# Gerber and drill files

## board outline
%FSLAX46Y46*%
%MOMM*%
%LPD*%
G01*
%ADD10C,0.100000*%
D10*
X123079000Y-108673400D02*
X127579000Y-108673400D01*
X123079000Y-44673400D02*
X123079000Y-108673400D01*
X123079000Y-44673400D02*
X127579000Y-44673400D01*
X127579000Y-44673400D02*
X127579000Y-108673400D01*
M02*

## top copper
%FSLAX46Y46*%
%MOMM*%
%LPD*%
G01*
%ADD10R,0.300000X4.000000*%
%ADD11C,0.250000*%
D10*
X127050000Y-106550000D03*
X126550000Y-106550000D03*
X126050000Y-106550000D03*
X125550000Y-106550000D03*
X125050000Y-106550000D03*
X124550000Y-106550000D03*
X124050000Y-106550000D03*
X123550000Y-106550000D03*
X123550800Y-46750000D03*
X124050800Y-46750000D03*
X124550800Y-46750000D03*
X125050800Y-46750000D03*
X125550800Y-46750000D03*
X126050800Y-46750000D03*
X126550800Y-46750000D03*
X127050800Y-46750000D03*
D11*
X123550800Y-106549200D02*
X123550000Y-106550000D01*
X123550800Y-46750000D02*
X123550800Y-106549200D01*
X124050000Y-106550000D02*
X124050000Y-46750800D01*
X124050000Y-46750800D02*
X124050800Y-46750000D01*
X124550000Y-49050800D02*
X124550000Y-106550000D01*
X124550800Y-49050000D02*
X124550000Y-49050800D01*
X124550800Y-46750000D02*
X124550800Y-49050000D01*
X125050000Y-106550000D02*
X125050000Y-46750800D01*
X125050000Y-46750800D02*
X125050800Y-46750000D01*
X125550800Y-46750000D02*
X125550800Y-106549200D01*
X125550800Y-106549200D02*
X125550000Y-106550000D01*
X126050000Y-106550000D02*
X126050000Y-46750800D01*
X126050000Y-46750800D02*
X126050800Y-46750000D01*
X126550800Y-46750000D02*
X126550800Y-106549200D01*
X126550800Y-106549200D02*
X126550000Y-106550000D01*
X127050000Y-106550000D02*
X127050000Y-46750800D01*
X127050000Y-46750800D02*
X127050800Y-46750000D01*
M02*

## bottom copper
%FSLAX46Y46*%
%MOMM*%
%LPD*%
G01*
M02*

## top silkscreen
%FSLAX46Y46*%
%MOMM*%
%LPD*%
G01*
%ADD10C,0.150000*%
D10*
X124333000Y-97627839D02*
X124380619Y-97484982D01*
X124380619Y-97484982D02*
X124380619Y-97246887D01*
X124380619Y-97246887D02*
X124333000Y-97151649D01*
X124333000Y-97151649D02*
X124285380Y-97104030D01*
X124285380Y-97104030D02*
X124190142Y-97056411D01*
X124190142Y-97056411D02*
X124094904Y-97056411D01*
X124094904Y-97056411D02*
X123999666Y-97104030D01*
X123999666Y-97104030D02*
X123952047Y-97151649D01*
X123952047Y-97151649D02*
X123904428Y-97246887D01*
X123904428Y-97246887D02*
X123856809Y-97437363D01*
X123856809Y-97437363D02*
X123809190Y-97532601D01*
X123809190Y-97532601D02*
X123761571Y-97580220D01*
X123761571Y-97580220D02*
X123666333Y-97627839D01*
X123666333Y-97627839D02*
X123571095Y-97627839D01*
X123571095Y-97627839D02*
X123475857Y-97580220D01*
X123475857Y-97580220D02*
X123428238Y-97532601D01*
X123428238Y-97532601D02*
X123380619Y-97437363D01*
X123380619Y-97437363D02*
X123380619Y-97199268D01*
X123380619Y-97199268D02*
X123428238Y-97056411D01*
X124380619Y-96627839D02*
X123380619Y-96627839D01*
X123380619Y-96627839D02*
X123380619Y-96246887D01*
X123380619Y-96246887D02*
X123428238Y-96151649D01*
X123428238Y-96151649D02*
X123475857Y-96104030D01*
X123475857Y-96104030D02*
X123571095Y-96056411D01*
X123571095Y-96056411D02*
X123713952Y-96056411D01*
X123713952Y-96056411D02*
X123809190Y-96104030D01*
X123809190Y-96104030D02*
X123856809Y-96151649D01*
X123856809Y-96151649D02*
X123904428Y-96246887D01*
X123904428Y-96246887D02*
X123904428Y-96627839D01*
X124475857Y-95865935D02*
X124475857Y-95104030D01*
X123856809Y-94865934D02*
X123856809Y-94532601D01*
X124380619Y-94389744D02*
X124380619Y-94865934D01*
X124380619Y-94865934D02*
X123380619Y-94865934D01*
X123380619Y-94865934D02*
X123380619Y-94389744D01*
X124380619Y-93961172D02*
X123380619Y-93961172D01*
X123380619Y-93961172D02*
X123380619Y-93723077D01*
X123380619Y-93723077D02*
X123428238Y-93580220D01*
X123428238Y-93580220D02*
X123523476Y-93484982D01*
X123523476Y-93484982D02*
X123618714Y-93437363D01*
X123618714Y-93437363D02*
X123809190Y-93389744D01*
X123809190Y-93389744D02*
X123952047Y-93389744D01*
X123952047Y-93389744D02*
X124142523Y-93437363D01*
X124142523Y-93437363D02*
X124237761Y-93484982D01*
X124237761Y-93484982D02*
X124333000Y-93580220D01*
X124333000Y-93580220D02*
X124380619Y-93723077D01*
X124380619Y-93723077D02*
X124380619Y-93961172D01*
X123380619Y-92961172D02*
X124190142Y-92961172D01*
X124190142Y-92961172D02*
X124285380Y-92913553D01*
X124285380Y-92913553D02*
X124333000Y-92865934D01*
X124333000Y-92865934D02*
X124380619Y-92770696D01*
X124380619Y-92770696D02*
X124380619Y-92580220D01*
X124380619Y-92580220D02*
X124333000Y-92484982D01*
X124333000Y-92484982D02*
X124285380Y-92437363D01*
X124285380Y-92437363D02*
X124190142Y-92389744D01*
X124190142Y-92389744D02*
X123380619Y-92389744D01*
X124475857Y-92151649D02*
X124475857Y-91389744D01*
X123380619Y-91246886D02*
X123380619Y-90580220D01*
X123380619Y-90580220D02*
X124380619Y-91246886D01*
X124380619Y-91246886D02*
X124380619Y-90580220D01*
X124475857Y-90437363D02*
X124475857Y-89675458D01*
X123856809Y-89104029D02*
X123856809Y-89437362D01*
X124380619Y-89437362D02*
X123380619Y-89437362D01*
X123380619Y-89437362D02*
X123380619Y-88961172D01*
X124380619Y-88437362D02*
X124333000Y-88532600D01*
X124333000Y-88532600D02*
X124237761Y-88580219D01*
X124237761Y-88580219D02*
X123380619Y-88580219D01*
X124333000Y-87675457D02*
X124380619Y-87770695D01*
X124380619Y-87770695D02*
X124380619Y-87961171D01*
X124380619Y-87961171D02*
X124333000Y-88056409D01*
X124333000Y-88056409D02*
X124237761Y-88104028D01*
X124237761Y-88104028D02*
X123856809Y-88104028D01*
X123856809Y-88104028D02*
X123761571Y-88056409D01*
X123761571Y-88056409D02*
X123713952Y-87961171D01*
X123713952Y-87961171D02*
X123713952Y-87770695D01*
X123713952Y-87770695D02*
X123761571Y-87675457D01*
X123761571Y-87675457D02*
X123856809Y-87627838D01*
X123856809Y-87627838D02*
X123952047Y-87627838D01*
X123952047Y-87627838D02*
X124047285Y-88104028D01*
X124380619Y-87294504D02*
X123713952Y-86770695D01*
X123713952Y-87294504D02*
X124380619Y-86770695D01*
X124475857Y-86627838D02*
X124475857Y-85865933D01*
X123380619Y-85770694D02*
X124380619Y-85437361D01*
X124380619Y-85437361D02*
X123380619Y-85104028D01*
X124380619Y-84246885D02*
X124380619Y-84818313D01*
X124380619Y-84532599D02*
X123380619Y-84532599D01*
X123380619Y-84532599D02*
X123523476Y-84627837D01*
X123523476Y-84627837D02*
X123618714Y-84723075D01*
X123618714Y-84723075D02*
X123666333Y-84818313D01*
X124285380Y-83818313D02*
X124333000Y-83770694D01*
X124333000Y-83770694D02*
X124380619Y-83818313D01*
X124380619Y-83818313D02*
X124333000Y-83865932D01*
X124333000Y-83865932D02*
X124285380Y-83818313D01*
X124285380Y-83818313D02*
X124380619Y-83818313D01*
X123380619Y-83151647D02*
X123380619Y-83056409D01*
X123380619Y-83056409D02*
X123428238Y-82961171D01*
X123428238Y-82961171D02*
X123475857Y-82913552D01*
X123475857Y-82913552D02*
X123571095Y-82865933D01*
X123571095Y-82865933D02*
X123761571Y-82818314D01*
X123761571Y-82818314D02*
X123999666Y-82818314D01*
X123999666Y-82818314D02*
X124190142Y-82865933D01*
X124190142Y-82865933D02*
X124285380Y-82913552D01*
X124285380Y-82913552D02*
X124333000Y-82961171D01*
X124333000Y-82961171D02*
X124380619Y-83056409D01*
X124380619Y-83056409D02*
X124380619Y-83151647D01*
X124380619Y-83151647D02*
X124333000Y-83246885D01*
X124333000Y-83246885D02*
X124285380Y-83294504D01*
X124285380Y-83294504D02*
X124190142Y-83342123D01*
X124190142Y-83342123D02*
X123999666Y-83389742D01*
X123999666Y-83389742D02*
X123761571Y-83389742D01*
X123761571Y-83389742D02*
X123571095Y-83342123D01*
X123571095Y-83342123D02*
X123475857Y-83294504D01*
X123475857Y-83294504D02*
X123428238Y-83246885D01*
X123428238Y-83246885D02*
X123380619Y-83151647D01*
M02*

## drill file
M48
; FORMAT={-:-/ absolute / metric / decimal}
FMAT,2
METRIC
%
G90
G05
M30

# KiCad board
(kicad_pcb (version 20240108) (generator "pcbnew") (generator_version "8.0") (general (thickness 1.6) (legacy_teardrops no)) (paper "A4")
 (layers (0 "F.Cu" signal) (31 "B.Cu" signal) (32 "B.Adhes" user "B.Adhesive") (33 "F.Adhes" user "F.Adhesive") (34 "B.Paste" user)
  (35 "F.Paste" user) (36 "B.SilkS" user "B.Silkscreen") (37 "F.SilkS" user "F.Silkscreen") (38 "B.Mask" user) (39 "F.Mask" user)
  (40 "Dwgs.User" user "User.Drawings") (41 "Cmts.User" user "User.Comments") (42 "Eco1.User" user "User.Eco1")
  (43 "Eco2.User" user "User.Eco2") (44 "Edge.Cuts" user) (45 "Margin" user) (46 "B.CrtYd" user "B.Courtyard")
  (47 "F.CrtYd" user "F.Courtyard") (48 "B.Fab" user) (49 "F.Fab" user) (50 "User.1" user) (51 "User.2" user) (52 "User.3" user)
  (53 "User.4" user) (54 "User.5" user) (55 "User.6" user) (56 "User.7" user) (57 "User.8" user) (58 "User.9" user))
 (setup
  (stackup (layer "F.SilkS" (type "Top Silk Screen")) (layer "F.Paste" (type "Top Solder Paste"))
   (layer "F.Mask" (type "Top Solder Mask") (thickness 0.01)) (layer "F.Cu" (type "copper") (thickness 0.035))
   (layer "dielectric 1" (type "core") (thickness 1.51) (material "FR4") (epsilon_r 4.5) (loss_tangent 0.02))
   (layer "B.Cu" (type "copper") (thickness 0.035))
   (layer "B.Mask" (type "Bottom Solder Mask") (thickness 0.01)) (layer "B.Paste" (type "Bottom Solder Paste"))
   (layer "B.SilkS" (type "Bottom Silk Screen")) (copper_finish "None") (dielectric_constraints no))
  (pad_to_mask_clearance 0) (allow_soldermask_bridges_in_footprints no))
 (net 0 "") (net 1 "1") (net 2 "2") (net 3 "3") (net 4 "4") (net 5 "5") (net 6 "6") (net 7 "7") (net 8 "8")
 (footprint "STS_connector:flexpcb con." (layer "F.Cu") (at 127.55 104.55 180)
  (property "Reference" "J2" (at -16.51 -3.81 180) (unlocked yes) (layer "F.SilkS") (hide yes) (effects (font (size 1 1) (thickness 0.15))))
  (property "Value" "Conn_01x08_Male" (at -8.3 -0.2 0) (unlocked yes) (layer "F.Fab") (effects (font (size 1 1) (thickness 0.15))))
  (pad "1" smd rect (at 0.5 -2 180) (size 0.3 4) (layers "F.Cu" "F.Paste" "F.Mask") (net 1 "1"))
  (pad "2" smd rect (at 1 -2 180) (size 0.3 4) (layers "F.Cu" "F.Paste" "F.Mask") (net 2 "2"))
  (pad "3" smd rect (at 1.5 -2 180) (size 0.3 4) (layers "F.Cu" "F.Paste" "F.Mask") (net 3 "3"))
  (pad "4" smd rect (at 2 -2 180) (size 0.3 4) (layers "F.Cu" "F.Paste" "F.Mask") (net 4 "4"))
  (pad "5" smd rect (at 2.5 -2 180) (size 0.3 4) (layers "F.Cu" "F.Paste" "F.Mask") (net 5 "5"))
  (pad "6" smd rect (at 3 -2 180) (size 0.3 4) (layers "F.Cu" "F.Paste" "F.Mask") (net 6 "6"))
  (pad "7" smd rect (at 3.5 -2 180) (size 0.3 4) (layers "F.Cu" "F.Paste" "F.Mask") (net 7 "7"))
  (pad "8" smd rect (at 4 -2 180) (size 0.3 4) (layers "F.Cu" "F.Paste" "F.Mask") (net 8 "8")))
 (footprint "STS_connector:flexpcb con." (layer "F.Cu") (at 123.0508 48.75)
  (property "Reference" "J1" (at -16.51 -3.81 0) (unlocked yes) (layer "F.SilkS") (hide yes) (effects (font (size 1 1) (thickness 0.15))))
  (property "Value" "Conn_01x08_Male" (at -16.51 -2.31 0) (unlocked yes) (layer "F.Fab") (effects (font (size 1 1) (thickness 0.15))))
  (pad "1" smd rect (at 0.5 -2) (size 0.3 4) (layers "F.Cu" "F.Paste" "F.Mask") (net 8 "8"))
  (pad "2" smd rect (at 1 -2) (size 0.3 4) (layers "F.Cu" "F.Paste" "F.Mask") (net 7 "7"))
  (pad "3" smd rect (at 1.5 -2) (size 0.3 4) (layers "F.Cu" "F.Paste" "F.Mask") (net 6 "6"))
  (pad "4" smd rect (at 2 -2) (size 0.3 4) (layers "F.Cu" "F.Paste" "F.Mask") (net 5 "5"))
  (pad "5" smd rect (at 2.5 -2) (size 0.3 4) (layers "F.Cu" "F.Paste" "F.Mask") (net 4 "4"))
  (pad "6" smd rect (at 3 -2) (size 0.3 4) (layers "F.Cu" "F.Paste" "F.Mask") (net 3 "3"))
  (pad "7" smd rect (at 3.5 -2) (size 0.3 4) (layers "F.Cu" "F.Paste" "F.Mask") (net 2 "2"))
  (pad "8" smd rect (at 4 -2) (size 0.3 4) (layers "F.Cu" "F.Paste" "F.Mask") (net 1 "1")))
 (gr_line (start 123.079 108.6734) (end 127.579 108.6734) (stroke (width 0.1) (type solid)) (layer "Edge.Cuts"))
 (gr_line (start 123.079 44.6734) (end 123.079 108.6734) (stroke (width 0.1) (type solid)) (layer "Edge.Cuts"))
 (gr_line (start 123.079 44.6734) (end 127.579 44.6734) (stroke (width 0.1) (type solid)) (layer "Edge.Cuts"))
 (gr_line (start 127.579 44.6734) (end 127.579 108.6734) (stroke (width 0.1) (type solid)) (layer "Edge.Cuts"))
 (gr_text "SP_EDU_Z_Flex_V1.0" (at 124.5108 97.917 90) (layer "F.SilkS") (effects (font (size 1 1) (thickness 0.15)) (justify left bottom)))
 (segment (start 123.5508 106.5492) (end 123.55 106.55) (width 0.25) (layer "F.Cu") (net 8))
 (segment (start 123.5508 46.75) (end 123.5508 106.5492) (width 0.25) (layer "F.Cu") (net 8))
 (segment (start 124.05 106.55) (end 124.05 46.7508) (width 0.25) (layer "F.Cu") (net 7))
 (segment (start 124.05 46.7508) (end 124.0508 46.75) (width 0.25) (layer "F.Cu") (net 7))
 (segment (start 124.55 49.0508) (end 124.55 106.55) (width 0.25) (layer "F.Cu") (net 6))
 (segment (start 124.5508 49.05) (end 124.55 49.0508) (width 0.25) (layer "F.Cu") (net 6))
 (segment (start 124.5508 46.75) (end 124.5508 49.05) (width 0.25) (layer "F.Cu") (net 6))
 (segment (start 125.05 106.55) (end 125.05 46.7508) (width 0.25) (layer "F.Cu") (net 5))
 (segment (start 125.05 46.7508) (end 125.0508 46.75) (width 0.25) (layer "F.Cu") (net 5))
 (segment (start 125.5508 46.75) (end 125.5508 106.5492) (width 0.25) (layer "F.Cu") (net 4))
 (segment (start 125.5508 106.5492) (end 125.55 106.55) (width 0.25) (layer "F.Cu") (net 4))
 (segment (start 126.05 106.55) (end 126.05 46.7508) (width 0.25) (layer "F.Cu") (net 3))
 (segment (start 126.05 46.7508) (end 126.0508 46.75) (width 0.25) (layer "F.Cu") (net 3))
 (segment (start 126.5508 46.75) (end 126.5508 106.5492) (width 0.25) (layer "F.Cu") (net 2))
 (segment (start 126.5508 106.5492) (end 126.55 106.55) (width 0.25) (layer "F.Cu") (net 2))
 (segment (start 127.05 106.55) (end 127.05 46.7508) (width 0.25) (layer "F.Cu") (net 1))
 (segment (start 127.05 46.7508) (end 127.0508 46.75) (width 0.25) (layer "F.Cu") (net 1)))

